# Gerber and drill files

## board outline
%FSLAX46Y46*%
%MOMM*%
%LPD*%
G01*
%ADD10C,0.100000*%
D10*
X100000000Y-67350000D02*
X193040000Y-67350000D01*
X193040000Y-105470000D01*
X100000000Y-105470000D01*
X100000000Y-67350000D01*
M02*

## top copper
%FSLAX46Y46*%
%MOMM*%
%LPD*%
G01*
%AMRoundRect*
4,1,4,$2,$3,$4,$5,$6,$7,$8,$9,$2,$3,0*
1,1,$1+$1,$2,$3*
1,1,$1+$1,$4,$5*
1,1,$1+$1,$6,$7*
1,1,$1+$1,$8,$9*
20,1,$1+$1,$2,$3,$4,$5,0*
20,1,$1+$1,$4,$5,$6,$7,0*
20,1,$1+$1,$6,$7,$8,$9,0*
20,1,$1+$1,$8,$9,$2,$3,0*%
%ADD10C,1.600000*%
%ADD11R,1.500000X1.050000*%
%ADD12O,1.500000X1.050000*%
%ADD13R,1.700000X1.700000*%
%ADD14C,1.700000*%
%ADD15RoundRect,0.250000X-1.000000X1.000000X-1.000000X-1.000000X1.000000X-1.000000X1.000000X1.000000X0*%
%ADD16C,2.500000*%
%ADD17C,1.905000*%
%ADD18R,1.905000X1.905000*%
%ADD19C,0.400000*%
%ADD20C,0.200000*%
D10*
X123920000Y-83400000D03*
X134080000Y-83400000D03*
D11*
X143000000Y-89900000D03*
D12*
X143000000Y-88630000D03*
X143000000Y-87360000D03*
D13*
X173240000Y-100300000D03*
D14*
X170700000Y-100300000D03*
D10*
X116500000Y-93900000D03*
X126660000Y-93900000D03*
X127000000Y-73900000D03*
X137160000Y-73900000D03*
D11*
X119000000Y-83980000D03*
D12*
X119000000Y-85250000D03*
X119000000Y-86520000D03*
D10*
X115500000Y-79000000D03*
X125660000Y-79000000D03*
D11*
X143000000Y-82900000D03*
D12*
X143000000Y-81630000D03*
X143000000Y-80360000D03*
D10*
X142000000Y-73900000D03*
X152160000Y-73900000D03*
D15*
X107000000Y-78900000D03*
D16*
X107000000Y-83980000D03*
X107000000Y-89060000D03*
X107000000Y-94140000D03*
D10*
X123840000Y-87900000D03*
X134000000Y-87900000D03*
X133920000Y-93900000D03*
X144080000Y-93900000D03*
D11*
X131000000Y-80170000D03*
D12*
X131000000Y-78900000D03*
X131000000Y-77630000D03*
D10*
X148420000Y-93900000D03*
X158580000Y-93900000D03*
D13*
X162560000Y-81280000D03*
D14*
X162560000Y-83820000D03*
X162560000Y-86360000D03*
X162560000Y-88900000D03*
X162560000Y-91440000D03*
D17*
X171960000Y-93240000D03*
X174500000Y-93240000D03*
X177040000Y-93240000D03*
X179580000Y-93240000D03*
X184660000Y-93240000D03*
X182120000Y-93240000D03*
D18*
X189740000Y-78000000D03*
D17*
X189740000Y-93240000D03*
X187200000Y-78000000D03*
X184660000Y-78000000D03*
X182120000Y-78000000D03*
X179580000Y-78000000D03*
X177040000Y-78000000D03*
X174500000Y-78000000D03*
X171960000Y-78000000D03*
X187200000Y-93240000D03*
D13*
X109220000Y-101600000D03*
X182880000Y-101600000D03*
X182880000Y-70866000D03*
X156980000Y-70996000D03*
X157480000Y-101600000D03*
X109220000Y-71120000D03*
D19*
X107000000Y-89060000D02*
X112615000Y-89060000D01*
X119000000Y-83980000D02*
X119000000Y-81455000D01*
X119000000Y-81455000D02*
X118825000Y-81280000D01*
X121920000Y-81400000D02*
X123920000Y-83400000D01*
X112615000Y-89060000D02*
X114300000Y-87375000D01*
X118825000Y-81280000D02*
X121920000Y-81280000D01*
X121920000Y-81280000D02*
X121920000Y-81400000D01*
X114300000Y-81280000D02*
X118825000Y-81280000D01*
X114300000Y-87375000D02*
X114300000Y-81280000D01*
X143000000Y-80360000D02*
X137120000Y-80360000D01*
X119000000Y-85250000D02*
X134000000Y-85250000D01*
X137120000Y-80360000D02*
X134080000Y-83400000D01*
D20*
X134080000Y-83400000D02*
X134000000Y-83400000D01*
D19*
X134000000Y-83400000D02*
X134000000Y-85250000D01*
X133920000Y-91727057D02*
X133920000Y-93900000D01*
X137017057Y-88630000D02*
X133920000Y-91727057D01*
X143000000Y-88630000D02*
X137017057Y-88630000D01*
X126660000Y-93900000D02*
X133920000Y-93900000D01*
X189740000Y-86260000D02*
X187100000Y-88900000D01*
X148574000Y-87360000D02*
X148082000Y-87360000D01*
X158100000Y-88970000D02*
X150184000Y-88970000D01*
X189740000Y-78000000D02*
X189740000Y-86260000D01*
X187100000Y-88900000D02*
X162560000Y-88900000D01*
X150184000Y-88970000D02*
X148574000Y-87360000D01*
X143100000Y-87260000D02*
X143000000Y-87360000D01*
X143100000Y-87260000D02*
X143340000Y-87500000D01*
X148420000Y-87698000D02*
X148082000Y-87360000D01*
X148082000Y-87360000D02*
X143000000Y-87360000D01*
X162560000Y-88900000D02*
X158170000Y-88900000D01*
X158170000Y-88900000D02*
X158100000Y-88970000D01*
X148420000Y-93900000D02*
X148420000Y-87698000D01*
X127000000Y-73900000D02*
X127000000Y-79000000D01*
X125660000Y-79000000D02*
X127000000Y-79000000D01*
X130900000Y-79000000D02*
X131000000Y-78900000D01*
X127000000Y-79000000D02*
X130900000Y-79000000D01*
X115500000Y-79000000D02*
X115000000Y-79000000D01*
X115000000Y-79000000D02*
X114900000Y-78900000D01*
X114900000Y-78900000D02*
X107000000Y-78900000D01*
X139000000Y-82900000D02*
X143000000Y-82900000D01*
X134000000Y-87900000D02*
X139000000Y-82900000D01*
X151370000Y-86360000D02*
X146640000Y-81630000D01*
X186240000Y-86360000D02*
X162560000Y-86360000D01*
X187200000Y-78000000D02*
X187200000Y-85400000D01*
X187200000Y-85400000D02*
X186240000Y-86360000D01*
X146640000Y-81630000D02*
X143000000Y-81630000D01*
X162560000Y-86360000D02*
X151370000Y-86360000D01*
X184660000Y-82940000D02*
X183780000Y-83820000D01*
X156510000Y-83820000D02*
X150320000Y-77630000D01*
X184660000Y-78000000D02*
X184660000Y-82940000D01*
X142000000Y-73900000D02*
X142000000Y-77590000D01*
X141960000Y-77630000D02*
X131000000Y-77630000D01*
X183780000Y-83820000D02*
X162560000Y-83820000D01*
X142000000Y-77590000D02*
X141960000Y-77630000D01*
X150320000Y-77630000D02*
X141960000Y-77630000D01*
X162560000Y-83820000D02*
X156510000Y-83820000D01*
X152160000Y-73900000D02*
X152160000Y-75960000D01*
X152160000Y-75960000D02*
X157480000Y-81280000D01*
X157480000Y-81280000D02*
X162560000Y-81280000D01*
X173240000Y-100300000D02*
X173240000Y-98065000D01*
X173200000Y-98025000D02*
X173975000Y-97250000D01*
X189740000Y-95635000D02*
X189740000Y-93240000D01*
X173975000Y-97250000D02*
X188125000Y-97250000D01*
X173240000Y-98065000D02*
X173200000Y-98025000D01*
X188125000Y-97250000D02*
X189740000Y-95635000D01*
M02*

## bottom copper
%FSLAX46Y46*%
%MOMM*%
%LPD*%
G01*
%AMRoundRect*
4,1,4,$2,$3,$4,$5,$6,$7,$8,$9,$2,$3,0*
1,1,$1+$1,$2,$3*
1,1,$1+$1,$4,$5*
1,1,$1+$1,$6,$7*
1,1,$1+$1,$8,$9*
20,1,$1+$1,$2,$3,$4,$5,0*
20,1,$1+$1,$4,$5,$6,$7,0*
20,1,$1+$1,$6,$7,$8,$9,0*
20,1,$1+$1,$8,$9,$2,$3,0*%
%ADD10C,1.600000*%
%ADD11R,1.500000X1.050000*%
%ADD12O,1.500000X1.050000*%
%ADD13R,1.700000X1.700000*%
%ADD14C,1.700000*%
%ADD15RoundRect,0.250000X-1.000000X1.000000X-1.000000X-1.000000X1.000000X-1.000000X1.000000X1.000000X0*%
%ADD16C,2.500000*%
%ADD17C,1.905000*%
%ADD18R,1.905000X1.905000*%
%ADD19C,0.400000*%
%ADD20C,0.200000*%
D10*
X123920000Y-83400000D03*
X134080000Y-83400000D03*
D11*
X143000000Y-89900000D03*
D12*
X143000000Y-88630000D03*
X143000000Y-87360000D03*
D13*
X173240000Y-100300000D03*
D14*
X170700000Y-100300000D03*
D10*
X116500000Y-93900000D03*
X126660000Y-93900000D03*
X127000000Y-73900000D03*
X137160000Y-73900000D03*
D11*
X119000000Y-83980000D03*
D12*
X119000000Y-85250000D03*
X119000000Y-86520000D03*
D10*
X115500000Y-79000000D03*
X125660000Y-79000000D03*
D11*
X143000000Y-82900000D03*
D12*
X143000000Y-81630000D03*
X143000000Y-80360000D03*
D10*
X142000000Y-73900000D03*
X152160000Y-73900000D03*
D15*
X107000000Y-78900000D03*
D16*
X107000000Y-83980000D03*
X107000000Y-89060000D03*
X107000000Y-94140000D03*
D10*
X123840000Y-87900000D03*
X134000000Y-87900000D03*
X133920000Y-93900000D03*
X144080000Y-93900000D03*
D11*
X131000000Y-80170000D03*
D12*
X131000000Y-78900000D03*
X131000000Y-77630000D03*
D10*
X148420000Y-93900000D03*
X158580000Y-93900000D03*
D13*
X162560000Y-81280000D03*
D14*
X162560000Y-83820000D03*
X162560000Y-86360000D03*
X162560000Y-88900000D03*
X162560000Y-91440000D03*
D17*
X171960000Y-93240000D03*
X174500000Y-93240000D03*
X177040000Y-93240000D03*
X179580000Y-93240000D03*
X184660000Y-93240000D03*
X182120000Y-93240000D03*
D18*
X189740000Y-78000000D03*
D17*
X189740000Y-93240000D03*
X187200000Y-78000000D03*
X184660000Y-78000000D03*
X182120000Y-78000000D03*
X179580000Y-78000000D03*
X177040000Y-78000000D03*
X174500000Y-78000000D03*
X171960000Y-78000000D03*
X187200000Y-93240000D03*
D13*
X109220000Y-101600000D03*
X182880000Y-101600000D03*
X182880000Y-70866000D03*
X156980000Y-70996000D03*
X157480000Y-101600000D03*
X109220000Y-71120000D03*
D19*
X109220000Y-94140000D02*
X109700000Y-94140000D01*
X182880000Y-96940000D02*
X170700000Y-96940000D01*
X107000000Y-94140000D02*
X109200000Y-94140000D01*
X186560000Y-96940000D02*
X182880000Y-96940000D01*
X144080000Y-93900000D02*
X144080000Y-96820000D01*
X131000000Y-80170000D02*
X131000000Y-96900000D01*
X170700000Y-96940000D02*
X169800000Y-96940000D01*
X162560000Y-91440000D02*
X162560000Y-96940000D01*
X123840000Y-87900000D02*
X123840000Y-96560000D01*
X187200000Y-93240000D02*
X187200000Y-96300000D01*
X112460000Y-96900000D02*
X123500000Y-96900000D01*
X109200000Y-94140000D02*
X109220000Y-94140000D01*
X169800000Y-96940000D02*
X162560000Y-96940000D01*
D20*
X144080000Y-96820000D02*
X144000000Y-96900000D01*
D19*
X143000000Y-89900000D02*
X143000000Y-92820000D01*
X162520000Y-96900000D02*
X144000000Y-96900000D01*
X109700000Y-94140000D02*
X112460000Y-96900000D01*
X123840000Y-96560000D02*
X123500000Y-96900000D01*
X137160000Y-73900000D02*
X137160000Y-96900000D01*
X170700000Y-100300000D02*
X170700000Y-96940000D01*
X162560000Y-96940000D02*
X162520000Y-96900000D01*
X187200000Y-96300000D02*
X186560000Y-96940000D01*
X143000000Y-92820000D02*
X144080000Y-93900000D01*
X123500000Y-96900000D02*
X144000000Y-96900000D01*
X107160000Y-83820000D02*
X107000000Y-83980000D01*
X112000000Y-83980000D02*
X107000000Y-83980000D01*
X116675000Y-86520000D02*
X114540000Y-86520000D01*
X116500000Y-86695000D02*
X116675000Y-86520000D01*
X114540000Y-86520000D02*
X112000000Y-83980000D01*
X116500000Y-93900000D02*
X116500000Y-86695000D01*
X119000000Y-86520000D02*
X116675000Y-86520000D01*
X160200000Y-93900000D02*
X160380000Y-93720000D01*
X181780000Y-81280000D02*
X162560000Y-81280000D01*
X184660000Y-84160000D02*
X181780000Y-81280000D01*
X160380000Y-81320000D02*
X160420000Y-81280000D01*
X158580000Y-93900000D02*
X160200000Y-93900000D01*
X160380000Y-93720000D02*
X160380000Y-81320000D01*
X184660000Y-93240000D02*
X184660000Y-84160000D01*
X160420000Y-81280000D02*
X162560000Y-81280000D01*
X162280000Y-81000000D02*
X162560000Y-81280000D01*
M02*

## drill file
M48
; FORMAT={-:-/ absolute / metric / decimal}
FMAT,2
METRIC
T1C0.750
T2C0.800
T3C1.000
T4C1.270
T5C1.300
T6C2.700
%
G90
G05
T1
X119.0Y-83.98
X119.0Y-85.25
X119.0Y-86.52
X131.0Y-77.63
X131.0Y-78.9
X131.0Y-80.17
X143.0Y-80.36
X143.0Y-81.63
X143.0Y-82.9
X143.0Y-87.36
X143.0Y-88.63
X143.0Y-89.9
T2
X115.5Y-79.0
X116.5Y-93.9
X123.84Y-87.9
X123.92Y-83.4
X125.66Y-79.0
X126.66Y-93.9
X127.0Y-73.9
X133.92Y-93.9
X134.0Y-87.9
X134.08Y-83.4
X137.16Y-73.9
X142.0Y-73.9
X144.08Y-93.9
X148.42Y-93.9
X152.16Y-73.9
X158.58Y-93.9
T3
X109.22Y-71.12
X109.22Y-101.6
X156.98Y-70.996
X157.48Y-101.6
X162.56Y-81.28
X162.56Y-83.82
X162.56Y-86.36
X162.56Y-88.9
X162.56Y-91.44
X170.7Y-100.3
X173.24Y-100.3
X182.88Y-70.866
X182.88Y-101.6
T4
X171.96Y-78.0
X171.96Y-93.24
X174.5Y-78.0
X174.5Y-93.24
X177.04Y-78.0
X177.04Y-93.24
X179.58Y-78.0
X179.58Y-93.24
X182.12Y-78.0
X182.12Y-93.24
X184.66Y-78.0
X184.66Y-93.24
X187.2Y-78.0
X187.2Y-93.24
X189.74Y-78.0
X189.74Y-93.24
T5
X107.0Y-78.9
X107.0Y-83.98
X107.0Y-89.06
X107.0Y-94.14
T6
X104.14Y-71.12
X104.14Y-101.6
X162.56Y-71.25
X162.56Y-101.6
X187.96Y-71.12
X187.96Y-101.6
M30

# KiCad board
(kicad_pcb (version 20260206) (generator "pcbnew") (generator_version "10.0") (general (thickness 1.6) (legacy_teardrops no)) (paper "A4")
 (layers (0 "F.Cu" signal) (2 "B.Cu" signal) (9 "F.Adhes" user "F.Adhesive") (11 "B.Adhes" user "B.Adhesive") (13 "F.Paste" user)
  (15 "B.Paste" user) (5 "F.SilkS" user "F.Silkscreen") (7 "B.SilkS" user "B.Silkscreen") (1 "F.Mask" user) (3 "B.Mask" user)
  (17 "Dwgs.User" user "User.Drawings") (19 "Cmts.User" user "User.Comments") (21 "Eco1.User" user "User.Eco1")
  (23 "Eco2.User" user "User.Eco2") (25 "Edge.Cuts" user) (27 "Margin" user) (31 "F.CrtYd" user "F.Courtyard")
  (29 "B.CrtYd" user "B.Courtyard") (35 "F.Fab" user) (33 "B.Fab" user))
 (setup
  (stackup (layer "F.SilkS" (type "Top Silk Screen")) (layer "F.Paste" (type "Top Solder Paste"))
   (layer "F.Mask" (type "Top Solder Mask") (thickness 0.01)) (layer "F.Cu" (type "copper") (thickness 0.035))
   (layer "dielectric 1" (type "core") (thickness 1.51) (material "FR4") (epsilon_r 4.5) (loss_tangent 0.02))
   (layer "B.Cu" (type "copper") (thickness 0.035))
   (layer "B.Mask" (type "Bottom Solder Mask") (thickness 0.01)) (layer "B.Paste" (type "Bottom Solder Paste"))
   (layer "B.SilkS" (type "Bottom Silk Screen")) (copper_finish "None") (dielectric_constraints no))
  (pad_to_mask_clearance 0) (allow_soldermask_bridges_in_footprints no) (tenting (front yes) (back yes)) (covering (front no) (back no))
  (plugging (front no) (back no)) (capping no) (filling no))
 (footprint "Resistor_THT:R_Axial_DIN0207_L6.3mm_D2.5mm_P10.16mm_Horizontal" (layer "F.Cu") (at 123.92 83.4)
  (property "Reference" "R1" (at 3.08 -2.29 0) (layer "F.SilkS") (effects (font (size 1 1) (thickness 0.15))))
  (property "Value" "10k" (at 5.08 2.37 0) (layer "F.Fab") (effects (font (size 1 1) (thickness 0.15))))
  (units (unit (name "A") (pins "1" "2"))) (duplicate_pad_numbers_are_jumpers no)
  (pad "1" thru_hole circle (at 0 0) (size 1.6 1.6) (drill 0.8) (layers "*.Cu" "*.Mask") (remove_unused_layers no) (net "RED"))
  (pad "2" thru_hole circle (at 10.16 0) (size 1.6 1.6) (drill 0.8) (layers "*.Cu" "*.Mask") (remove_unused_layers no) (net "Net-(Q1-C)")))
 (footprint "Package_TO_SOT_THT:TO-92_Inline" (layer "F.Cu") (at 143 89.9 90)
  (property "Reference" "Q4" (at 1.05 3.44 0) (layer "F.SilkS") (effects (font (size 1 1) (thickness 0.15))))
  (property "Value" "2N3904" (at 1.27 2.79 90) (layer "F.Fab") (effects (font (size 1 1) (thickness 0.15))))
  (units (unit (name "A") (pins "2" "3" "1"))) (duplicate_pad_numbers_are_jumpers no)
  (pad "1" thru_hole rect (at 0 0 90) (size 1.05 1.5) (drill 0.75) (layers "*.Cu" "*.Mask") (remove_unused_layers no) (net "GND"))
  (pad "2" thru_hole oval (at 1.27 0 90) (size 1.05 1.5) (drill 0.75) (layers "*.Cu" "*.Mask") (remove_unused_layers no) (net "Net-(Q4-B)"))
  (pad "3" thru_hole oval (at 2.54 0 90) (size 1.05 1.5) (drill 0.75) (layers "*.Cu" "*.Mask") (remove_unused_layers no) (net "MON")))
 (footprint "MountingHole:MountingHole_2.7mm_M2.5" (layer "F.Cu") (at 187.96 101.6)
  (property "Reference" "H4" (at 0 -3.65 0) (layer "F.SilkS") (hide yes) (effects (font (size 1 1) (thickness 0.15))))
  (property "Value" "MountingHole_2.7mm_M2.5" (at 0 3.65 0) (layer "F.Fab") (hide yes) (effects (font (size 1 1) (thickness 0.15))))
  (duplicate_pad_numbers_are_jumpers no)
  (pad "" np_thru_hole circle (at 0 0) (size 2.7 2.7) (drill 2.7) (layers "*.Cu" "*.Mask")))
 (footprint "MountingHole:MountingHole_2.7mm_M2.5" (layer "F.Cu") (at 162.56 101.6)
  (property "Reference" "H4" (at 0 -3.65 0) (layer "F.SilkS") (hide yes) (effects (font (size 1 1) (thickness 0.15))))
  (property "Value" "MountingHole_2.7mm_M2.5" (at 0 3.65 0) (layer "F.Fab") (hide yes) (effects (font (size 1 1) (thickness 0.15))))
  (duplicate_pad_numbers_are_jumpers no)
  (pad "" np_thru_hole circle (at 0 0) (size 2.7 2.7) (drill 2.7) (layers "*.Cu" "*.Mask")))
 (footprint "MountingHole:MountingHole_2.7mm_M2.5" (layer "F.Cu") (at 104.14 71.12)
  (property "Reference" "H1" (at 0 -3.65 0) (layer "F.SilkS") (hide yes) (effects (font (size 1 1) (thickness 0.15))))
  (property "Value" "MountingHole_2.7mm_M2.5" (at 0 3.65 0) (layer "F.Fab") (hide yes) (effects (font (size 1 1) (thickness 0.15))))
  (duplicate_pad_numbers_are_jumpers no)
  (pad "" np_thru_hole circle (at 0 0) (size 2.7 2.7) (drill 2.7) (layers "*.Cu" "*.Mask")))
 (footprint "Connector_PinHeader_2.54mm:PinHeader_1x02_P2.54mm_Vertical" (layer "F.Cu") (at 173.24 100.3 -90)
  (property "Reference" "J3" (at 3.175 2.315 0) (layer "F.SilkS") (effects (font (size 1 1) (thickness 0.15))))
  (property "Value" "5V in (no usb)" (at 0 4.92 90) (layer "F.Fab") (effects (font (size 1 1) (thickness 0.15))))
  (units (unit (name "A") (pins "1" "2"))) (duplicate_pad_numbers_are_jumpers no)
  (pad "1" thru_hole rect (at 0 0 270) (size 1.7 1.7) (drill 1) (layers "*.Cu" "*.Mask") (remove_unused_layers no) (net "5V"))
  (pad "2" thru_hole circle (at 0 2.54 270) (size 1.7 1.7) (drill 1) (layers "*.Cu" "*.Mask") (remove_unused_layers no) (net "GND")))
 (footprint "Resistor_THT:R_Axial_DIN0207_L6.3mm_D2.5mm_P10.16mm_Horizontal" (layer "F.Cu") (at 116.5 93.9)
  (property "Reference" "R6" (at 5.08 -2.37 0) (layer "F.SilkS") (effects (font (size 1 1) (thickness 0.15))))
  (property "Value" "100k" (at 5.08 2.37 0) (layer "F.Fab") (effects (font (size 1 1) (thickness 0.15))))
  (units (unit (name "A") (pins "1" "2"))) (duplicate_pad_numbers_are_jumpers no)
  (pad "1" thru_hole circle (at 0 0) (size 1.6 1.6) (drill 0.8) (layers "*.Cu" "*.Mask") (remove_unused_layers no) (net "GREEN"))
  (pad "2" thru_hole circle (at 10.16 0) (size 1.6 1.6) (drill 0.8) (layers "*.Cu" "*.Mask") (remove_unused_layers no) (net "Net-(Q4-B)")))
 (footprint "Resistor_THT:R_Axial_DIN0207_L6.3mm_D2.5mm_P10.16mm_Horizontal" (layer "F.Cu") (at 127 73.9)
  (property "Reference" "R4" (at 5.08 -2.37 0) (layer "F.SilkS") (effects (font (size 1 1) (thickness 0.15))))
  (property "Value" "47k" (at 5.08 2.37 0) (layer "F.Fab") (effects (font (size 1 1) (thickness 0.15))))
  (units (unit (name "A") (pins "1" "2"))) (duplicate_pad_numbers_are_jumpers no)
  (pad "1" thru_hole circle (at 0 0) (size 1.6 1.6) (drill 0.8) (layers "*.Cu" "*.Mask") (remove_unused_layers no) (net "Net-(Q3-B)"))
  (pad "2" thru_hole circle (at 10.16 0) (size 1.6 1.6) (drill 0.8) (layers "*.Cu" "*.Mask") (remove_unused_layers no) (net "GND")))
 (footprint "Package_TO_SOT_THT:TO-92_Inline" (layer "F.Cu") (at 119 83.98 -90)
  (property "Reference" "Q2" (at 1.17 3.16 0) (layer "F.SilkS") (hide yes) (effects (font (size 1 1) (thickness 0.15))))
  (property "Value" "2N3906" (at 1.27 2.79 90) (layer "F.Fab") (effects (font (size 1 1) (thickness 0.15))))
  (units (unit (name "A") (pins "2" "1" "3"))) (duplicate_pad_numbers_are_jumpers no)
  (pad "1" thru_hole rect (at 0 0 270) (size 1.05 1.5) (drill 0.75) (layers "*.Cu" "*.Mask") (remove_unused_layers no) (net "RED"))
  (pad "2" thru_hole oval (at 1.27 0 270) (size 1.05 1.5) (drill 0.75) (layers "*.Cu" "*.Mask") (remove_unused_layers no) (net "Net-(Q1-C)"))
  (pad "3" thru_hole oval (at 2.54 0 270) (size 1.05 1.5) (drill 0.75) (layers "*.Cu" "*.Mask") (remove_unused_layers no) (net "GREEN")))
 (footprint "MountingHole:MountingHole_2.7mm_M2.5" (layer "F.Cu") (at 162.56 71.25)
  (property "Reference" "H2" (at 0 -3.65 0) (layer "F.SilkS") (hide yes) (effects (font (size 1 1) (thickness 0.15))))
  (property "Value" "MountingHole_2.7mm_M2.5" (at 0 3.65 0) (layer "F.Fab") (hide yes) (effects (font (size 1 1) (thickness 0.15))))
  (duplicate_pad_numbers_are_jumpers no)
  (pad "" np_thru_hole circle (at 0 0) (size 2.7 2.7) (drill 2.7) (layers "*.Cu" "*.Mask")))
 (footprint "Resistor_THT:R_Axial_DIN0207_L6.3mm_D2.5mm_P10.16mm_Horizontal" (layer "F.Cu") (at 115.5 79)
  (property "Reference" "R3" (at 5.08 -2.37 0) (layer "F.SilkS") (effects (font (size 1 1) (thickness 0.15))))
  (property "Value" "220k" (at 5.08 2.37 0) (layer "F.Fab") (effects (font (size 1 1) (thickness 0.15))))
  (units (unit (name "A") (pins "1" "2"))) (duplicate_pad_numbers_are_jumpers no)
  (pad "1" thru_hole circle (at 0 0) (size 1.6 1.6) (drill 0.8) (layers "*.Cu" "*.Mask") (remove_unused_layers no) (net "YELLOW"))
  (pad "2" thru_hole circle (at 10.16 0) (size 1.6 1.6) (drill 0.8) (layers "*.Cu" "*.Mask") (remove_unused_layers no) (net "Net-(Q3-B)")))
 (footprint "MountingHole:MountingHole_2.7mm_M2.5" (layer "F.Cu") (at 187.96 71.12)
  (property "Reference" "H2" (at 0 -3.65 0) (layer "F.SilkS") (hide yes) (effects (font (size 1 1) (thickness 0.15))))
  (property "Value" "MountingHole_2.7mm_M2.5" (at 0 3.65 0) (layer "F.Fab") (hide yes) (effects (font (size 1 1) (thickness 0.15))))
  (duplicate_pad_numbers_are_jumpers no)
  (pad "" np_thru_hole circle (at 0 0) (size 2.7 2.7) (drill 2.7) (layers "*.Cu" "*.Mask")))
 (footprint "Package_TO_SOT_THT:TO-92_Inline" (layer "F.Cu") (at 143 82.9 90)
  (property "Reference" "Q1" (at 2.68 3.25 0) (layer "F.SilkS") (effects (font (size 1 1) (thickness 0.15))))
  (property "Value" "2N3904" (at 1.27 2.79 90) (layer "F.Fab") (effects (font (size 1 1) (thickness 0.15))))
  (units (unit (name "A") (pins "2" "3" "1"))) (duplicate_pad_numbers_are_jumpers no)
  (pad "1" thru_hole rect (at 0 0 90) (size 1.05 1.5) (drill 0.75) (layers "*.Cu" "*.Mask") (remove_unused_layers no) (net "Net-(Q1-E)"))
  (pad "2" thru_hole oval (at 1.27 0 90) (size 1.05 1.5) (drill 0.75) (layers "*.Cu" "*.Mask") (remove_unused_layers no) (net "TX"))
  (pad "3" thru_hole oval (at 2.54 0 90) (size 1.05 1.5) (drill 0.75) (layers "*.Cu" "*.Mask") (remove_unused_layers no) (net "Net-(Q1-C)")))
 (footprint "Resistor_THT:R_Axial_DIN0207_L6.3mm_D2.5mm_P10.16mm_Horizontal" (layer "F.Cu") (at 142 73.9)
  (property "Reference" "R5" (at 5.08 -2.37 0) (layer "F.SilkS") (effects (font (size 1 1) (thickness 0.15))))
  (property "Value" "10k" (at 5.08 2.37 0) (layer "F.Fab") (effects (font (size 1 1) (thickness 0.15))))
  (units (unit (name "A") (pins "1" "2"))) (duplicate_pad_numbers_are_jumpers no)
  (pad "1" thru_hole circle (at 0 0) (size 1.6 1.6) (drill 0.8) (layers "*.Cu" "*.Mask") (remove_unused_layers no) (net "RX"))
  (pad "2" thru_hole circle (at 10.16 0) (size 1.6 1.6) (drill 0.8) (layers "*.Cu" "*.Mask") (remove_unused_layers no) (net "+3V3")))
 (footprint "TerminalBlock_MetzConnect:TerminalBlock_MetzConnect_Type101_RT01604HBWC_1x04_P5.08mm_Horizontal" (layer "F.Cu")
  (at 107 78.9 -90)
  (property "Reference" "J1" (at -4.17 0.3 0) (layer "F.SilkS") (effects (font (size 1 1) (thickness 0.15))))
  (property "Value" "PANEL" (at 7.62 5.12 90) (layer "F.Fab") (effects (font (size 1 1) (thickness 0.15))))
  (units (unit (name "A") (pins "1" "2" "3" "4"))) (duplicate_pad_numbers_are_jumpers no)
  (pad "1" thru_hole roundrect (at 0 0 270) (size 2.5 2.5) (drill 1.3) (layers "*.Cu" "*.Mask") (remove_unused_layers no)
   (roundrect_rratio 0.1) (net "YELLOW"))
  (pad "2" thru_hole circle (at 5.08 0 270) (size 2.5 2.5) (drill 1.3) (layers "*.Cu" "*.Mask") (remove_unused_layers no) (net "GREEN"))
  (pad "3" thru_hole circle (at 10.16 0 270) (size 2.5 2.5) (drill 1.3) (layers "*.Cu" "*.Mask") (remove_unused_layers no) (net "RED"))
  (pad "4" thru_hole circle (at 15.24 0 270) (size 2.5 2.5) (drill 1.3) (layers "*.Cu" "*.Mask") (remove_unused_layers no) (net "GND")))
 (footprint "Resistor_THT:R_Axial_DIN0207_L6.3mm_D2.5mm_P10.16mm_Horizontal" (layer "F.Cu") (at 123.84 87.9)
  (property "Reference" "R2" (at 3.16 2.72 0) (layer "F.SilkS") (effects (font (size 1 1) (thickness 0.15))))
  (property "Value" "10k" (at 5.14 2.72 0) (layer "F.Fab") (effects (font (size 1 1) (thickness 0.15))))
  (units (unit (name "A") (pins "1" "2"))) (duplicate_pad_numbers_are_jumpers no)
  (pad "1" thru_hole circle (at 0 0) (size 1.6 1.6) (drill 0.8) (layers "*.Cu" "*.Mask") (remove_unused_layers no) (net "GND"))
  (pad "2" thru_hole circle (at 10.16 0) (size 1.6 1.6) (drill 0.8) (layers "*.Cu" "*.Mask") (remove_unused_layers no) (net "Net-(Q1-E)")))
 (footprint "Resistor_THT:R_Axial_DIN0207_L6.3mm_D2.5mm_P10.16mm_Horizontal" (layer "F.Cu") (at 133.92 93.9)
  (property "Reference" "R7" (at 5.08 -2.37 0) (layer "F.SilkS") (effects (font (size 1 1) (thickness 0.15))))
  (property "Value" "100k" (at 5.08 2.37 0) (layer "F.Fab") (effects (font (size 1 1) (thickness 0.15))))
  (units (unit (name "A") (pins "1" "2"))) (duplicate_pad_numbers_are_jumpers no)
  (pad "1" thru_hole circle (at 0 0) (size 1.6 1.6) (drill 0.8) (layers "*.Cu" "*.Mask") (remove_unused_layers no) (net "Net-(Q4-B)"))
  (pad "2" thru_hole circle (at 10.16 0) (size 1.6 1.6) (drill 0.8) (layers "*.Cu" "*.Mask") (remove_unused_layers no) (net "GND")))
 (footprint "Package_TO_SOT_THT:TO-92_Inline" (layer "F.Cu") (at 131 80.17 90)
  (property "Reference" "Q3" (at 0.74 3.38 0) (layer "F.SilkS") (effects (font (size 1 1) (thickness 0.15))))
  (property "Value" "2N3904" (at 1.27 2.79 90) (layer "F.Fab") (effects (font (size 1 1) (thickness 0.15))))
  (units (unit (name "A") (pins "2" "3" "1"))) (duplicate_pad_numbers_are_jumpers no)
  (pad "1" thru_hole rect (at 0 0 90) (size 1.05 1.5) (drill 0.75) (layers "*.Cu" "*.Mask") (remove_unused_layers no) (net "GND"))
  (pad "2" thru_hole oval (at 1.27 0 90) (size 1.05 1.5) (drill 0.75) (layers "*.Cu" "*.Mask") (remove_unused_layers no) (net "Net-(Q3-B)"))
  (pad "3" thru_hole oval (at 2.54 0 90) (size 1.05 1.5) (drill 0.75) (layers "*.Cu" "*.Mask") (remove_unused_layers no) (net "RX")))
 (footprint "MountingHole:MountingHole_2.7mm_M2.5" (layer "F.Cu") (at 104.14 101.6)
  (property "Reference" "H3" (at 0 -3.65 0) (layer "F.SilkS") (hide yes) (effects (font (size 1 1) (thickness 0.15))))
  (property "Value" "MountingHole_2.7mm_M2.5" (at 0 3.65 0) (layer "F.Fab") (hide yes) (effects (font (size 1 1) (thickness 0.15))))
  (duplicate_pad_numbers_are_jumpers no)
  (pad "" np_thru_hole circle (at 0 0) (size 2.7 2.7) (drill 2.7) (layers "*.Cu" "*.Mask")))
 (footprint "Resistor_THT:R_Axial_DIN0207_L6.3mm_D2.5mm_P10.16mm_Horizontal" (layer "F.Cu") (at 148.42 93.9)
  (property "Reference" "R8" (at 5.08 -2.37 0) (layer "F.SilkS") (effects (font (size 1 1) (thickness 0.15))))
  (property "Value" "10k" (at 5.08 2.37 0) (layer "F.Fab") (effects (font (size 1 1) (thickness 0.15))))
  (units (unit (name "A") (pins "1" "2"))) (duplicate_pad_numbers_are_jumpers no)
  (pad "1" thru_hole circle (at 0 0) (size 1.6 1.6) (drill 0.8) (layers "*.Cu" "*.Mask") (remove_unused_layers no) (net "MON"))
  (pad "2" thru_hole circle (at 10.16 0) (size 1.6 1.6) (drill 0.8) (layers "*.Cu" "*.Mask") (remove_unused_layers no) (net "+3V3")))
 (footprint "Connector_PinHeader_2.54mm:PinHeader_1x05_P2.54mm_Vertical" (layer "F.Cu") (at 162.56 81.28)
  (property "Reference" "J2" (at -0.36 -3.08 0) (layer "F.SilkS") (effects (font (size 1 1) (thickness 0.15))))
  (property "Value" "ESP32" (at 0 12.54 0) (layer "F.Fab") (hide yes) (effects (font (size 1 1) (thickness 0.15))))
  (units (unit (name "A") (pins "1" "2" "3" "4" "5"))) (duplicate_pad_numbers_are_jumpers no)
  (pad "1" thru_hole rect (at 0 0) (size 1.7 1.7) (drill 1) (layers "*.Cu" "*.Mask") (remove_unused_layers no) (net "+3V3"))
  (pad "2" thru_hole circle (at 0 2.54) (size 1.7 1.7) (drill 1) (layers "*.Cu" "*.Mask") (remove_unused_layers no) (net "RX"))
  (pad "3" thru_hole circle (at 0 5.08) (size 1.7 1.7) (drill 1) (layers "*.Cu" "*.Mask") (remove_unused_layers no) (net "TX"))
  (pad "4" thru_hole circle (at 0 7.62) (size 1.7 1.7) (drill 1) (layers "*.Cu" "*.Mask") (remove_unused_layers no) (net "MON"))
  (pad "5" thru_hole circle (at 0 10.16) (size 1.7 1.7) (drill 1) (layers "*.Cu" "*.Mask") (remove_unused_layers no) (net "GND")))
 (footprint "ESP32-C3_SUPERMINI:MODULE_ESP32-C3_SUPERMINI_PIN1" (layer "F.Cu") (at 179.84 85.62 -90)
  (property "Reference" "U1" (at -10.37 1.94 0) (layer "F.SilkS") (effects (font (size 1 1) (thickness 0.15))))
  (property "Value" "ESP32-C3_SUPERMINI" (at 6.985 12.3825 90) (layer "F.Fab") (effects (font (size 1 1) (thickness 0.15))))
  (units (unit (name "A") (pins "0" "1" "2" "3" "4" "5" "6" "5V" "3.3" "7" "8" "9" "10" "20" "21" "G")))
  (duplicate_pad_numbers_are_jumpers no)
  (pad "0" thru_hole circle (at 7.62 7.88 270) (size 1.905 1.905) (drill 1.27) (layers "*.Cu" "*.Mask") (remove_unused_layers no)
   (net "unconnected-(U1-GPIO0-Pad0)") (solder_mask_margin 0.102))
  (pad "1" thru_hole circle (at 7.62 5.34 270) (size 1.905 1.905) (drill 1.27) (layers "*.Cu" "*.Mask") (remove_unused_layers no)
   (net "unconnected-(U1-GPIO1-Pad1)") (solder_mask_margin 0.102))
  (pad "2" thru_hole circle (at 7.62 2.8 270) (size 1.905 1.905) (drill 1.27) (layers "*.Cu" "*.Mask") (remove_unused_layers no)
   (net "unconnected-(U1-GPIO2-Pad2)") (solder_mask_margin 0.102))
  (pad "3" thru_hole circle (at 7.62 0.26 270) (size 1.905 1.905) (drill 1.27) (layers "*.Cu" "*.Mask") (remove_unused_layers no)
   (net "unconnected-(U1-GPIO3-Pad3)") (solder_mask_margin 0.102))
  (pad "3.3" thru_hole circle (at 7.62 -4.82 270) (size 1.905 1.905) (drill 1.27) (layers "*.Cu" "*.Mask") (remove_unused_layers no)
   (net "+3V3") (solder_mask_margin 0.102))
  (pad "4" thru_hole circle (at 7.62 -2.28 270) (size 1.905 1.905) (drill 1.27) (layers "*.Cu" "*.Mask") (remove_unused_layers no)
   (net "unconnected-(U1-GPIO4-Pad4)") (solder_mask_margin 0.102))
  (pad "5" thru_hole rect (at -7.62 -9.9 270) (size 1.905 1.905) (drill 1.27) (layers "*.Cu" "*.Mask") (remove_unused_layers no) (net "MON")
   (solder_mask_margin 0.102))
  (pad "5V" thru_hole circle (at 7.62 -9.9 270) (size 1.905 1.905) (drill 1.27) (layers "*.Cu" "*.Mask") (remove_unused_layers no)
   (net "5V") (solder_mask_margin 0.102))
  (pad "6" thru_hole circle (at -7.62 -7.36 270) (size 1.905 1.905) (drill 1.27) (layers "*.Cu" "*.Mask") (remove_unused_layers no)
   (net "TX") (solder_mask_margin 0.102))
  (pad "7" thru_hole circle (at -7.62 -4.82 270) (size 1.905 1.905) (drill 1.27) (layers "*.Cu" "*.Mask") (remove_unused_layers no)
   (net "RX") (solder_mask_margin 0.102))
  (pad "8" thru_hole circle (at -7.62 -2.28 270) (size 1.905 1.905) (drill 1.27) (layers "*.Cu" "*.Mask") (remove_unused_layers no)
   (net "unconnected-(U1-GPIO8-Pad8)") (solder_mask_margin 0.102))
  (pad "9" thru_hole circle (at -7.62 0.26 270) (size 1.905 1.905) (drill 1.27) (layers "*.Cu" "*.Mask") (remove_unused_layers no)
   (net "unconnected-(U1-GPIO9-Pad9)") (solder_mask_margin 0.102))
  (pad "10" thru_hole circle (at -7.62 2.8 270) (size 1.905 1.905) (drill 1.27) (layers "*.Cu" "*.Mask") (remove_unused_layers no)
   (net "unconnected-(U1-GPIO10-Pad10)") (solder_mask_margin 0.102))
  (pad "20" thru_hole circle (at -7.62 5.34 270) (size 1.905 1.905) (drill 1.27) (layers "*.Cu" "*.Mask") (remove_unused_layers no)
   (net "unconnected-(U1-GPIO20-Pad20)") (solder_mask_margin 0.102))
  (pad "21" thru_hole circle (at -7.62 7.88 270) (size 1.905 1.905) (drill 1.27) (layers "*.Cu" "*.Mask") (remove_unused_layers no)
   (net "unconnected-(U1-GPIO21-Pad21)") (solder_mask_margin 0.102))
  (pad "G" thru_hole circle (at 7.62 -7.36 270) (size 1.905 1.905) (drill 1.27) (layers "*.Cu" "*.Mask") (remove_unused_layers no)
   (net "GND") (solder_mask_margin 0.102)))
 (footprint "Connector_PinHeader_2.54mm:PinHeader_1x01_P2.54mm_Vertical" (layer "B.Cu") (at 109.22 101.6)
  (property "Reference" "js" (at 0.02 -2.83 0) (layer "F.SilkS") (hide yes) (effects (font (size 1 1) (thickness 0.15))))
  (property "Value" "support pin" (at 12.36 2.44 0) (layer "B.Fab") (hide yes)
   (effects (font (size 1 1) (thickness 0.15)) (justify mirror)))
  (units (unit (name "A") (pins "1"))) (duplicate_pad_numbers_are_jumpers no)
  (pad "1" thru_hole rect (at 0 0) (size 1.7 1.7) (drill 1) (layers "*.Cu" "*.Mask") (remove_unused_layers no)
   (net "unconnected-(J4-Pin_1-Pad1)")))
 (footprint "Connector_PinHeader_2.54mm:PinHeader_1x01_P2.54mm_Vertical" (layer "B.Cu") (at 182.88 101.6)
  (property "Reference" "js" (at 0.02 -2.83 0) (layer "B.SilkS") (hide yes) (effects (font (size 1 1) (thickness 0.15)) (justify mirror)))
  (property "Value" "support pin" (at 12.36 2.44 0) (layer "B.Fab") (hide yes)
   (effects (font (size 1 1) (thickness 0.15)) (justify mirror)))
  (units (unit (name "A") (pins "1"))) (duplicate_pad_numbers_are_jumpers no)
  (pad "1" thru_hole rect (at 0 0) (size 1.7 1.7) (drill 1) (layers "*.Cu" "*.Mask") (remove_unused_layers no)
   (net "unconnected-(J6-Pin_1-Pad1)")))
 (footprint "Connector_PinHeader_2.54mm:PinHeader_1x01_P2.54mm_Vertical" (layer "B.Cu") (at 182.88 70.866)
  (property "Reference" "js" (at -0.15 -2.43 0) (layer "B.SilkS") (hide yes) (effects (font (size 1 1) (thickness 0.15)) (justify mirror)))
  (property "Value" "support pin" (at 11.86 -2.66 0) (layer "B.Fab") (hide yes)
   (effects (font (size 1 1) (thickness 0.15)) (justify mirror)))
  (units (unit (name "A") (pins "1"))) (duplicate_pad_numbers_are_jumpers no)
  (pad "1" thru_hole rect (at 0 0) (size 1.7 1.7) (drill 1) (layers "*.Cu" "*.Mask") (remove_unused_layers no)
   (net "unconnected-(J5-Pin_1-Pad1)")))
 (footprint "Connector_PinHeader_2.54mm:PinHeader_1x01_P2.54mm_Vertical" (layer "B.Cu") (at 156.98 70.996)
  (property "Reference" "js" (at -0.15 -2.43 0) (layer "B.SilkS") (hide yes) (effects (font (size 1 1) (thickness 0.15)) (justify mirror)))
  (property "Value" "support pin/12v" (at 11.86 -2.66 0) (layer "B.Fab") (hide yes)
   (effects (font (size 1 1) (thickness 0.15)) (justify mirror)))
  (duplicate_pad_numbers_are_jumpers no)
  (pad "1" thru_hole rect (at 0 0) (size 1.7 1.7) (drill 1) (layers "*.Cu" "*.Mask") (remove_unused_layers no)))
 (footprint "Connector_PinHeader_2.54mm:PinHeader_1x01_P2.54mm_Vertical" (layer "B.Cu") (at 157.48 101.6)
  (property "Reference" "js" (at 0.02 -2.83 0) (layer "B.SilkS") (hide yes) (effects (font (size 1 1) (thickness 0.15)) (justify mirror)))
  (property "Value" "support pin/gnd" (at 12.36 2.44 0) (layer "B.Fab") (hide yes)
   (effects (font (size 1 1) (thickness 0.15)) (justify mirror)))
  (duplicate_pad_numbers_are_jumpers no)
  (pad "1" thru_hole rect (at 0 0) (size 1.7 1.7) (drill 1) (layers "*.Cu" "*.Mask") (remove_unused_layers no)))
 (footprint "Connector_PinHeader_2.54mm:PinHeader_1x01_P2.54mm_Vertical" (layer "B.Cu") (at 109.22 71.12)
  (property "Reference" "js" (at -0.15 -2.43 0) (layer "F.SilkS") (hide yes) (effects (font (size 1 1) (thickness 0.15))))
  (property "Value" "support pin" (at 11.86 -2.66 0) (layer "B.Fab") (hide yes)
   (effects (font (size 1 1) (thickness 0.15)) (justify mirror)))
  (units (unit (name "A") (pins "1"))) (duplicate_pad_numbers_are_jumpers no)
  (pad "1" thru_hole rect (at 0 0) (size 1.7 1.7) (drill 1) (layers "*.Cu" "*.Mask") (remove_unused_layers no)
   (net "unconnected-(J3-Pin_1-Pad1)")))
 (gr_rect (start 100 67.35) (end 193.04 105.47) (stroke (width 0.1) (type default)) (fill no) (layer "Edge.Cuts"))
 (segment (start 107 89.06) (end 112.615 89.06) (width 0.4) (layer "F.Cu") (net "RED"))
 (segment (start 119 83.98) (end 119 81.455) (width 0.4) (layer "F.Cu") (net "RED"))
 (segment (start 119 81.455) (end 118.825 81.28) (width 0.4) (layer "F.Cu") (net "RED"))
 (segment (start 121.92 81.4) (end 123.92 83.4) (width 0.4) (layer "F.Cu") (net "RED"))
 (segment (start 112.615 89.06) (end 114.3 87.375) (width 0.4) (layer "F.Cu") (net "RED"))
 (segment (start 118.825 81.28) (end 121.92 81.28) (width 0.4) (layer "F.Cu") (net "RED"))
 (segment (start 121.92 81.28) (end 121.92 81.4) (width 0.4) (layer "F.Cu") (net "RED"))
 (segment (start 114.3 81.28) (end 118.825 81.28) (width 0.4) (layer "F.Cu") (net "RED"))
 (segment (start 114.3 87.375) (end 114.3 81.28) (width 0.4) (layer "F.Cu") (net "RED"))
 (segment (start 143 80.36) (end 137.12 80.36) (width 0.4) (layer "F.Cu") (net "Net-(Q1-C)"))
 (segment (start 119 85.25) (end 134 85.25) (width 0.4) (layer "F.Cu") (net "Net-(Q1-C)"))
 (segment (start 137.12 80.36) (end 134.08 83.4) (width 0.4) (layer "F.Cu") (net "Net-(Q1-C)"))
 (segment (start 134.08 83.4) (end 134 83.4) (width 0.2) (layer "F.Cu") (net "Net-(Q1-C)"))
 (segment (start 134 83.4) (end 134 85.25) (width 0.4) (layer "F.Cu") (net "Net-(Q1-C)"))
 (segment (start 109.22 94.14) (end 109.7 94.14) (width 0.4) (layer "B.Cu") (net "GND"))
 (segment (start 182.88 96.94) (end 170.7 96.94) (width 0.4) (layer "B.Cu") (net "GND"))
 (segment (start 107 94.14) (end 109.2 94.14) (width 0.4) (layer "B.Cu") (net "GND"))
 (segment (start 186.56 96.94) (end 182.88 96.94) (width 0.4) (layer "B.Cu") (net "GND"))
 (segment (start 144.08 93.9) (end 144.08 96.82) (width 0.4) (layer "B.Cu") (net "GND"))
 (segment (start 131 80.17) (end 131 96.9) (width 0.4) (layer "B.Cu") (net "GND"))
 (segment (start 170.7 96.94) (end 169.8 96.94) (width 0.4) (layer "B.Cu") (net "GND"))
 (segment (start 162.56 91.44) (end 162.56 96.94) (width 0.4) (layer "B.Cu") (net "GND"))
 (segment (start 123.84 87.9) (end 123.84 96.56) (width 0.4) (layer "B.Cu") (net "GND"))
 (segment (start 187.2 93.24) (end 187.2 96.3) (width 0.4) (layer "B.Cu") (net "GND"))
 (segment (start 112.46 96.9) (end 123.5 96.9) (width 0.4) (layer "B.Cu") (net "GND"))
 (segment (start 109.2 94.14) (end 109.22 94.14) (width 0.4) (layer "B.Cu") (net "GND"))
 (segment (start 169.8 96.94) (end 162.56 96.94) (width 0.4) (layer "B.Cu") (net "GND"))
 (segment (start 144.08 96.82) (end 144 96.9) (width 0.2) (layer "B.Cu") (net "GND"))
 (segment (start 143 89.9) (end 143 92.82) (width 0.4) (layer "B.Cu") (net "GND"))
 (segment (start 162.52 96.9) (end 144 96.9) (width 0.4) (layer "B.Cu") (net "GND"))
 (segment (start 109.7 94.14) (end 112.46 96.9) (width 0.4) (layer "B.Cu") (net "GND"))
 (segment (start 123.84 96.56) (end 123.5 96.9) (width 0.4) (layer "B.Cu") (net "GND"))
 (segment (start 137.16 73.9) (end 137.16 96.9) (width 0.4) (layer "B.Cu") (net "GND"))
 (segment (start 170.7 100.3) (end 170.7 96.94) (width 0.4) (layer "B.Cu") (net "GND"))
 (segment (start 162.56 96.94) (end 162.52 96.9) (width 0.4) (layer "B.Cu") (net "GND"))
 (segment (start 187.2 96.3) (end 186.56 96.94) (width 0.4) (layer "B.Cu") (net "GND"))
 (segment (start 143 92.82) (end 144.08 93.9) (width 0.4) (layer "B.Cu") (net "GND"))
 (segment (start 123.5 96.9) (end 144 96.9) (width 0.4) (layer "B.Cu") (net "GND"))
 (segment (start 133.92 91.727057) (end 133.92 93.9) (width 0.4) (layer "F.Cu") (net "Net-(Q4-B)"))
 (segment (start 137.017057 88.63) (end 133.92 91.727057) (width 0.4) (layer "F.Cu") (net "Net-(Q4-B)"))
 (segment (start 143 88.63) (end 137.017057 88.63) (width 0.4) (layer "F.Cu") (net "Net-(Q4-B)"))
 (segment (start 126.66 93.9) (end 133.92 93.9) (width 0.4) (layer "F.Cu") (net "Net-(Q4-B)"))
 (segment (start 189.74 86.26) (end 187.1 88.9) (width 0.4) (layer "F.Cu") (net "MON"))
 (segment (start 148.574 87.36) (end 148.082 87.36) (width 0.4) (layer "F.Cu") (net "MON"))
 (segment (start 158.1 88.97) (end 150.184 88.97) (width 0.4) (layer "F.Cu") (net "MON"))
 (segment (start 189.74 78) (end 189.74 86.26) (width 0.4) (layer "F.Cu") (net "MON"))
 (segment (start 187.1 88.9) (end 162.56 88.9) (width 0.4) (layer "F.Cu") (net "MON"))
 (segment (start 150.184 88.97) (end 148.574 87.36) (width 0.4) (layer "F.Cu") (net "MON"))
 (segment (start 143.1 87.26) (end 143 87.36) (width 0.4) (layer "F.Cu") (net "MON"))
 (segment (start 143.1 87.26) (end 143.34 87.5) (width 0.4) (layer "F.Cu") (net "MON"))
 (segment (start 148.42 87.698) (end 148.082 87.36) (width 0.4) (layer "F.Cu") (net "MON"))
 (segment (start 148.082 87.36) (end 143 87.36) (width 0.4) (layer "F.Cu") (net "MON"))
 (segment (start 162.56 88.9) (end 158.17 88.9) (width 0.4) (layer "F.Cu") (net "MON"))
 (segment (start 158.17 88.9) (end 158.1 88.97) (width 0.4) (layer "F.Cu") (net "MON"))
 (segment (start 148.42 93.9) (end 148.42 87.698) (width 0.4) (layer "F.Cu") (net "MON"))
 (segment (start 107.16 83.82) (end 107 83.98) (width 0.4) (layer "B.Cu") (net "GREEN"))
 (segment (start 112 83.98) (end 107 83.98) (width 0.4) (layer "B.Cu") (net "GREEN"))
 (segment (start 116.675 86.52) (end 114.54 86.52) (width 0.4) (layer "B.Cu") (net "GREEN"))
 (segment (start 116.5 86.695) (end 116.675 86.52) (width 0.4) (layer "B.Cu") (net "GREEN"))
 (segment (start 114.54 86.52) (end 112 83.98) (width 0.4) (layer "B.Cu") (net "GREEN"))
 (segment (start 116.5 93.9) (end 116.5 86.695) (width 0.4) (layer "B.Cu") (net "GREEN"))
 (segment (start 119 86.52) (end 116.675 86.52) (width 0.4) (layer "B.Cu") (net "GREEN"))
 (segment (start 127 73.9) (end 127 79) (width 0.4) (layer "F.Cu") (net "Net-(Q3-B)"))
 (segment (start 125.66 79) (end 127 79) (width 0.4) (layer "F.Cu") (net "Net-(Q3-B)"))
 (segment (start 130.9 79) (end 131 78.9) (width 0.4) (layer "F.Cu") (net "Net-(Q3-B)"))
 (segment (start 127 79) (end 130.9 79) (width 0.4) (layer "F.Cu") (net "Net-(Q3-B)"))
 (segment (start 115.5 79) (end 115 79) (width 0.4) (layer "F.Cu") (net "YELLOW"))
 (segment (start 115 79) (end 114.9 78.9) (width 0.4) (layer "F.Cu") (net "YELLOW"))
 (segment (start 114.9 78.9) (end 107 78.9) (width 0.4) (layer "F.Cu") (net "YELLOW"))
 (segment (start 139 82.9) (end 143 82.9) (width 0.4) (layer "F.Cu") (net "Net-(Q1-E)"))
 (segment (start 134 87.9) (end 139 82.9) (width 0.4) (layer "F.Cu") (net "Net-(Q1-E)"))
 (segment (start 151.37 86.36) (end 146.64 81.63) (width 0.4) (layer "F.Cu") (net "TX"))
 (segment (start 186.24 86.36) (end 162.56 86.36) (width 0.4) (layer "F.Cu") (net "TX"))
 (segment (start 187.2 78) (end 187.2 85.4) (width 0.4) (layer "F.Cu") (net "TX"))
 (segment (start 187.2 85.4) (end 186.24 86.36) (width 0.4) (layer "F.Cu") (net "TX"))
 (segment (start 146.64 81.63) (end 143 81.63) (width 0.4) (layer "F.Cu") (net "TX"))
 (segment (start 162.56 86.36) (end 151.37 86.36) (width 0.4) (layer "F.Cu") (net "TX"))
 (segment (start 184.66 82.94) (end 183.78 83.82) (width 0.4) (layer "F.Cu") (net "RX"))
 (segment (start 156.51 83.82) (end 150.32 77.63) (width 0.4) (layer "F.Cu") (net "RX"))
 (segment (start 184.66 78) (end 184.66 82.94) (width 0.4) (layer "F.Cu") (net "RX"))
 (segment (start 142 73.9) (end 142 77.59) (width 0.4) (layer "F.Cu") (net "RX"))
 (segment (start 141.96 77.63) (end 131 77.63) (width 0.4) (layer "F.Cu") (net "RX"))
 (segment (start 183.78 83.82) (end 162.56 83.82) (width 0.4) (layer "F.Cu") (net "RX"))
 (segment (start 142 77.59) (end 141.96 77.63) (width 0.4) (layer "F.Cu") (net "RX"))
 (segment (start 150.32 77.63) (end 141.96 77.63) (width 0.4) (layer "F.Cu") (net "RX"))
 (segment (start 162.56 83.82) (end 156.51 83.82) (width 0.4) (layer "F.Cu") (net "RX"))
 (segment (start 152.16 73.9) (end 152.16 75.96) (width 0.4) (layer "F.Cu") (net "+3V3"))
 (segment (start 152.16 75.96) (end 157.48 81.28) (width 0.4) (layer "F.Cu") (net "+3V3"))
 (segment (start 157.48 81.28) (end 162.56 81.28) (width 0.4) (layer "F.Cu") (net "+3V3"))
 (segment (start 160.2 93.9) (end 160.38 93.72) (width 0.4) (layer "B.Cu") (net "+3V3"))
 (segment (start 181.78 81.28) (end 162.56 81.28) (width 0.4) (layer "B.Cu") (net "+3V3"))
 (segment (start 184.66 84.16) (end 181.78 81.28) (width 0.4) (layer "B.Cu") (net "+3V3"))
 (segment (start 160.38 81.32) (end 160.42 81.28) (width 0.4) (layer "B.Cu") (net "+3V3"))
 (segment (start 158.58 93.9) (end 160.2 93.9) (width 0.4) (layer "B.Cu") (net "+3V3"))
 (segment (start 160.38 93.72) (end 160.38 81.32) (width 0.4) (layer "B.Cu") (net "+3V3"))
 (segment (start 184.66 93.24) (end 184.66 84.16) (width 0.4) (layer "B.Cu") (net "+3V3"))
 (segment (start 160.42 81.28) (end 162.56 81.28) (width 0.4) (layer "B.Cu") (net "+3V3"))
 (segment (start 162.28 81) (end 162.56 81.28) (width 0.4) (layer "B.Cu") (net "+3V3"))
 (segment (start 173.24 100.3) (end 173.24 98.065) (width 0.4) (layer "F.Cu") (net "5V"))
 (segment (start 173.2 98.025) (end 173.975 97.25) (width 0.4) (layer "F.Cu") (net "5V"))
 (segment (start 189.74 95.635) (end 189.74 93.24) (width 0.4) (layer "F.Cu") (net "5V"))
 (segment (start 173.975 97.25) (end 188.125 97.25) (width 0.4) (layer "F.Cu") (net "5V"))
 (segment (start 173.24 98.065) (end 173.2 98.025) (width 0.4) (layer "F.Cu") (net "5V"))
 (segment (start 188.125 97.25) (end 189.74 95.635) (width 0.4) (layer "F.Cu") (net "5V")))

